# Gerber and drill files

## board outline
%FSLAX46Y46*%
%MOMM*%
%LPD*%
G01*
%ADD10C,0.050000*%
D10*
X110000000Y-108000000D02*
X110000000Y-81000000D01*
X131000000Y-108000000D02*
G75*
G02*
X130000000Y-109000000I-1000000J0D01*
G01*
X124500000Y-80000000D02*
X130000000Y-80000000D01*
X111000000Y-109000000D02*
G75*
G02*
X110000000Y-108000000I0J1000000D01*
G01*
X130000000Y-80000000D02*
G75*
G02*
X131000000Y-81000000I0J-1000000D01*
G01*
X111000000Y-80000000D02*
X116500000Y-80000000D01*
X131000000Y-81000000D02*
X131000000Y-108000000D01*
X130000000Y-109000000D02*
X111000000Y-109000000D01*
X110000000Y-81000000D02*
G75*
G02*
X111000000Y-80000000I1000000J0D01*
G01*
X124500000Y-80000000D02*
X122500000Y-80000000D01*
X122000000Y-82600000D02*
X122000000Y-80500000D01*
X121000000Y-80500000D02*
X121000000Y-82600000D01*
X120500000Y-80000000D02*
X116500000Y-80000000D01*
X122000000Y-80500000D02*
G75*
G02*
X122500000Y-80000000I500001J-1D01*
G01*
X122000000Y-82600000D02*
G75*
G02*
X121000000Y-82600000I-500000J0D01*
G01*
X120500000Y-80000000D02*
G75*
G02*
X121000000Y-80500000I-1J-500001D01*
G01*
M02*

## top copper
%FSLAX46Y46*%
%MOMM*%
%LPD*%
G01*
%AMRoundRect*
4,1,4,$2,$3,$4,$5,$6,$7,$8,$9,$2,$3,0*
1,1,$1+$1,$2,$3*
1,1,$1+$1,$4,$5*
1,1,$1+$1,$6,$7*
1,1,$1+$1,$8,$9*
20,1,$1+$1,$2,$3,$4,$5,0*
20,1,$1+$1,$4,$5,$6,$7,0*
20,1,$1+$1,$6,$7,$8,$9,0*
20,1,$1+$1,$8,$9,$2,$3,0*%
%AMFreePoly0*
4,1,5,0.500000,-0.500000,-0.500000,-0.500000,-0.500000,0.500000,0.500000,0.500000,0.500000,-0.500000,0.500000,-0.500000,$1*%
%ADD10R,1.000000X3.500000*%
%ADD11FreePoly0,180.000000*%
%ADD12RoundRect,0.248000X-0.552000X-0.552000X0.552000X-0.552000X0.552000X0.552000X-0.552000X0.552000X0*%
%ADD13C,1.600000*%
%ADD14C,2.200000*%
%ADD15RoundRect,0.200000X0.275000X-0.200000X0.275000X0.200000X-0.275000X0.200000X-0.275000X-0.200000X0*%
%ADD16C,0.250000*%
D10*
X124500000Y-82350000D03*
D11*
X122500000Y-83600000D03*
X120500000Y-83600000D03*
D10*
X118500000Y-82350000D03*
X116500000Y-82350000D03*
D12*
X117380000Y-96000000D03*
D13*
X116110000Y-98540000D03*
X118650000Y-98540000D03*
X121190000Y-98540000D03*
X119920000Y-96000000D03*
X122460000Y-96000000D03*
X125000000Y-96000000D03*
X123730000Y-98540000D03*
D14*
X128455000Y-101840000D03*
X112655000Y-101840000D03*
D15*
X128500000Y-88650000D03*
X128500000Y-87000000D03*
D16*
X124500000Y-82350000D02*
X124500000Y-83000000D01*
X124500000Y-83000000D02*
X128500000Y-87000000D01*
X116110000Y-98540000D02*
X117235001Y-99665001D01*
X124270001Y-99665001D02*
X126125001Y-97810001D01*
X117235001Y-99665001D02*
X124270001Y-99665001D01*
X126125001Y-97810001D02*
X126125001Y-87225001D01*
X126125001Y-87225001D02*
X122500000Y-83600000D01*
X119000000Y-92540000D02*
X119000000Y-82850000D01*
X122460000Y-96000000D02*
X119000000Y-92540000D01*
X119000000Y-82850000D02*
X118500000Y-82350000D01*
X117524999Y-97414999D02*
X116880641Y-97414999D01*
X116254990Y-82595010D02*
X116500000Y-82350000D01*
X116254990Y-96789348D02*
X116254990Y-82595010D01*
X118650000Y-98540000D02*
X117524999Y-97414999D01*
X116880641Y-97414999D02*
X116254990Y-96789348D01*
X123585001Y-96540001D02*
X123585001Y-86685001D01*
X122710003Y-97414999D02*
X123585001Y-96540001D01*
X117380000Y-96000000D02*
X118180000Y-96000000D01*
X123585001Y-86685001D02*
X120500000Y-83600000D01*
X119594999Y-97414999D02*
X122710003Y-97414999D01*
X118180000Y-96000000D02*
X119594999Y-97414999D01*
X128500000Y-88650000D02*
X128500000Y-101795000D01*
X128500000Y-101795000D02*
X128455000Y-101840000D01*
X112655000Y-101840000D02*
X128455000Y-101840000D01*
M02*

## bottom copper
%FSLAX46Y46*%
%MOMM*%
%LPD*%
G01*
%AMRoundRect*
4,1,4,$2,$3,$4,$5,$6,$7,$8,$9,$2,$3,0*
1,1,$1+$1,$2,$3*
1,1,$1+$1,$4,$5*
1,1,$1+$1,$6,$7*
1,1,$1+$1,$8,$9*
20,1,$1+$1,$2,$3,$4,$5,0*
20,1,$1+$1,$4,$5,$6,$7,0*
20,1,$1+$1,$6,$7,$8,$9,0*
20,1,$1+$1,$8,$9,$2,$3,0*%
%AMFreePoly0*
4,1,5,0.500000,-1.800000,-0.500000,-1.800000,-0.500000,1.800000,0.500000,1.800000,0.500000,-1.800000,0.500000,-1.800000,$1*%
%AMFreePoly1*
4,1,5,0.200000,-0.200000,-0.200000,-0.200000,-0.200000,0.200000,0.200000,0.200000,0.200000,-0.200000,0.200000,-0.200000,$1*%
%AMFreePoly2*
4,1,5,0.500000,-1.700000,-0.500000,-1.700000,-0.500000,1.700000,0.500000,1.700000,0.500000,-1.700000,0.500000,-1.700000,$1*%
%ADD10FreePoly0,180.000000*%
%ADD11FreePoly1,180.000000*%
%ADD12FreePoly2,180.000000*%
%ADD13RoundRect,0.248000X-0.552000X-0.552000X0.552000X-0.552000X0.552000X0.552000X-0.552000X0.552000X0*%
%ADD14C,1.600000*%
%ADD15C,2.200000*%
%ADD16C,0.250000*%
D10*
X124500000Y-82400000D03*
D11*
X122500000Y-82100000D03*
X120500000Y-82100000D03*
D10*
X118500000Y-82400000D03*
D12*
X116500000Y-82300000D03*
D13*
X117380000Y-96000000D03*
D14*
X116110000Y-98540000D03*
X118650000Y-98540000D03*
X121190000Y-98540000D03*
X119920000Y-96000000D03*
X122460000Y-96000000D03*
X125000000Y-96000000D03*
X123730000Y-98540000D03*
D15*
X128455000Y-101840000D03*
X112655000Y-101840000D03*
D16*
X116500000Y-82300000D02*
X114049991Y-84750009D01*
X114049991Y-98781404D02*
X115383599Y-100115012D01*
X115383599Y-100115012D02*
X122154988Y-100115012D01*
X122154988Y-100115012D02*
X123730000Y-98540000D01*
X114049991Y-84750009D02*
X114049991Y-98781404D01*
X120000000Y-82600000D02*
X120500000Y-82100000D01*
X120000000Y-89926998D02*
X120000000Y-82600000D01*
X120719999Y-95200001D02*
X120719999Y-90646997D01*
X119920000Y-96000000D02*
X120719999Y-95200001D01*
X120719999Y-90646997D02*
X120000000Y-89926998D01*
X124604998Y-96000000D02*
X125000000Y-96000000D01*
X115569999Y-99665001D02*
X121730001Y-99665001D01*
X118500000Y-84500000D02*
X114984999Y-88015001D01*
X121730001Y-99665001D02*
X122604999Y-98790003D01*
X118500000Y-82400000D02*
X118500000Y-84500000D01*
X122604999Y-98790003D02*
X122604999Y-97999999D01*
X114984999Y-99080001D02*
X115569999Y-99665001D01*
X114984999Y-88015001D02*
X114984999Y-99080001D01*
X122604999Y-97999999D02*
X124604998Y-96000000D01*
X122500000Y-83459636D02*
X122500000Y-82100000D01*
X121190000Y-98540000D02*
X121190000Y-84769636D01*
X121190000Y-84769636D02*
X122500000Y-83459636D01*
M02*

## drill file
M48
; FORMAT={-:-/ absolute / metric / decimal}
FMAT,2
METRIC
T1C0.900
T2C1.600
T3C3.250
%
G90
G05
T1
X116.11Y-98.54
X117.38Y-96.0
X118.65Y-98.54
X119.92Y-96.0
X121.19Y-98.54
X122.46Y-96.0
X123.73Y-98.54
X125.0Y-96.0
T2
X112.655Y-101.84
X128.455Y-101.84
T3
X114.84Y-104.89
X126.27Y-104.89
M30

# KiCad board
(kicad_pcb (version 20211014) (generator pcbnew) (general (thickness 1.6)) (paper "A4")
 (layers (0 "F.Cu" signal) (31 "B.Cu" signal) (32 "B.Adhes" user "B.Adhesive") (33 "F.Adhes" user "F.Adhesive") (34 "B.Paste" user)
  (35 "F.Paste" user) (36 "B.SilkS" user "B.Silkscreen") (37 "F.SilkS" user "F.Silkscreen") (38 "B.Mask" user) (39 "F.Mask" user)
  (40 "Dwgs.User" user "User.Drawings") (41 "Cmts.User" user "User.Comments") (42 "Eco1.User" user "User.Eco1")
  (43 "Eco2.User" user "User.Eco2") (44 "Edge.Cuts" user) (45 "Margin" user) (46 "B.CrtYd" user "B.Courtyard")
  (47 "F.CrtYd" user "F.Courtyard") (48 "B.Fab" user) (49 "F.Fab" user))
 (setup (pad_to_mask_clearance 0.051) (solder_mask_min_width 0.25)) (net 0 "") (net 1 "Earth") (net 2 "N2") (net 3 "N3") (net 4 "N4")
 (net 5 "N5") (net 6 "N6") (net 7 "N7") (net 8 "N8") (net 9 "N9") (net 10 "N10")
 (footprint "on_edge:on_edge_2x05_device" (layer "F.Cu") (at 120.5 80 180)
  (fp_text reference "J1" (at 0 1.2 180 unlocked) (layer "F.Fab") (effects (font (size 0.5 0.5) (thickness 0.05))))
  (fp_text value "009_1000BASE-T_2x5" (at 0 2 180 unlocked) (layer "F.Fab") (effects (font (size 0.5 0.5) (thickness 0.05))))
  (fp_line (start -4 0) (end -2 0) (layer "Edge.Cuts") (width 0.05))
  (fp_line (start -1.5 -2.6) (end -1.5 -0.5) (layer "Edge.Cuts") (width 0.05))
  (fp_line (start -0.5 -0.5) (end -0.5 -2.6) (layer "Edge.Cuts") (width 0.05))
  (fp_line (start 0 0) (end 4 0) (layer "Edge.Cuts") (width 0.05))
  (fp_arc (start -1.5 -0.5) (mid -1.646447 -0.146447) (end -2 0) (layer "Edge.Cuts") (width 0.05))
  (fp_arc (start -1.5 -2.6) (mid -1 -3.1) (end -0.5 -2.6) (layer "Edge.Cuts") (width 0.05))
  (fp_arc (start 0 0) (mid -0.353553 -0.146447) (end -0.5 -0.5) (layer "Edge.Cuts") (width 0.05))
  (pad "1" smd rect locked (at -4 -2.35) (size 1 3.5) (layers "F.Cu" "F.Mask") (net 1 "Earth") (zone_connect 0))
  (pad "2" smd custom locked (at -2 -3.6 180) (size 1 1) (layers "F.Cu" "F.Mask") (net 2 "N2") (zone_connect 0)
   (options (clearance outline) (anchor rect)) (primitives))
  (pad "3" smd custom locked (at 0 -3.6 180) (size 1 1) (layers "F.Cu" "F.Mask") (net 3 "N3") (zone_connect 0)
   (options (clearance outline) (anchor rect)) (primitives))
  (pad "4" smd rect locked (at 2 -2.35) (size 1 3.5) (layers "F.Cu" "F.Mask") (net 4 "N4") (zone_connect 0))
  (pad "5" smd rect locked (at 4 -2.35) (size 1 3.5) (layers "F.Cu" "F.Mask") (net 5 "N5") (zone_connect 0))
  (pad "6" smd custom locked (at -4 -2.4 180) (size 1 3.6) (layers "B.Cu" "B.Mask") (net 1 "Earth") (zone_connect 0)
   (options (clearance outline) (anchor rect)) (primitives))
  (pad "7" smd custom locked (at -2 -2.1 180) (size 0.4 0.4) (layers "B.Cu" "B.Mask") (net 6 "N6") (zone_connect 0)
   (options (clearance outline) (anchor rect)) (primitives))
  (pad "8" smd custom locked (at 0 -2.1 180) (size 0.4 0.4) (layers "B.Cu" "B.Mask") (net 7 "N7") (zone_connect 0)
   (options (clearance outline) (anchor rect)) (primitives))
  (pad "9" smd custom locked (at 2 -2.4 180) (size 1 3.6) (layers "B.Cu" "B.Mask") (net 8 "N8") (zone_connect 0)
   (options (clearance outline) (anchor rect)) (primitives))
  (pad "10" smd custom locked (at 4 -2.3 180) (size 1 3.4) (layers "B.Cu" "B.Mask") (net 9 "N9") (zone_connect 0)
   (options (clearance outline) (anchor rect)) (primitives)))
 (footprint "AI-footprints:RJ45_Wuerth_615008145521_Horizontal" (layer "F.Cu") (at 125 96 -90)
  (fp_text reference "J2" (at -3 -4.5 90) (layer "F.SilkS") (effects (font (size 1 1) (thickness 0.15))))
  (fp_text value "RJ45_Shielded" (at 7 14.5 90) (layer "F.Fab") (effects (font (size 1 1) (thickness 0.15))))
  (pad "" np_thru_hole circle locked (at 8.89 10.16) (size 3.25 3.25) (drill 3.25) (layers *.Cu *.Mask))
  (pad "" np_thru_hole circle locked (at 8.89 -1.27) (size 3.25 3.25) (drill 3.25) (layers *.Cu *.Mask))
  (pad "1" thru_hole roundrect locked (at 0 7.62) (size 1.6 1.6) (drill 0.9) (layers *.Cu *.Mask) (roundrect_rratio 0.155) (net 3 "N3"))
  (pad "2" thru_hole circle locked (at 2.54 8.89) (size 1.6 1.6) (drill 0.9) (layers *.Cu *.Mask) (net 2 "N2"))
  (pad "3" thru_hole circle locked (at 2.54 6.35) (size 1.6 1.6) (drill 0.9) (layers *.Cu *.Mask) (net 5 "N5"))
  (pad "4" thru_hole circle locked (at 2.54 3.81) (size 1.6 1.6) (drill 0.9) (layers *.Cu *.Mask) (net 6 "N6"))
  (pad "5" thru_hole circle locked (at 0 5.08) (size 1.6 1.6) (drill 0.9) (layers *.Cu *.Mask) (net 7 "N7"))
  (pad "6" thru_hole circle locked (at 0 2.54) (size 1.6 1.6) (drill 0.9) (layers *.Cu *.Mask) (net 4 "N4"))
  (pad "7" thru_hole circle locked (at 0 0) (size 1.6 1.6) (drill 0.9) (layers *.Cu *.Mask) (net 8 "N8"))
  (pad "8" thru_hole circle locked (at 2.54 1.27) (size 1.6 1.6) (drill 0.9) (layers *.Cu *.Mask) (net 9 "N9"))
  (pad "SH" thru_hole circle locked (at 5.84 -3.455) (size 2.2 2.2) (drill 1.6) (layers *.Cu *.Mask) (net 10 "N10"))
  (pad "SH" thru_hole circle locked (at 5.84 12.345) (size 2.2 2.2) (drill 1.6) (layers *.Cu *.Mask) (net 10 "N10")))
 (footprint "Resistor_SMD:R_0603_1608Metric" (layer "F.Cu") (at 128.5 87.825 90)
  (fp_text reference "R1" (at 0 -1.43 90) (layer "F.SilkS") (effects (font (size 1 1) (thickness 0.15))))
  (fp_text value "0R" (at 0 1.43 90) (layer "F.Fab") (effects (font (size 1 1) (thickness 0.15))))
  (pad "1" smd roundrect locked (at -0.825 0 90) (size 0.8 0.95) (layers "F.Cu" "F.Paste" "F.Mask") (roundrect_rratio 0.25) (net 10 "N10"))
  (pad "2" smd roundrect locked (at 0.825 0 90) (size 0.8 0.95) (layers "F.Cu" "F.Paste" "F.Mask") (roundrect_rratio 0.25) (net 1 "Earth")))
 (gr_line (start 110 108) (end 110 81) (layer "Edge.Cuts") (width 0.05))
 (gr_arc (start 131 108) (mid 130.707107 108.707107) (end 130 109) (layer "Edge.Cuts") (width 0.05))
 (gr_line (start 124.5 80) (end 130 80) (layer "Edge.Cuts") (width 0.05))
 (gr_arc (start 111 109) (mid 110.292893 108.707107) (end 110 108) (layer "Edge.Cuts") (width 0.05))
 (gr_arc (start 130 80) (mid 130.707107 80.292893) (end 131 81) (layer "Edge.Cuts") (width 0.05))
 (gr_line (start 111 80) (end 116.5 80) (layer "Edge.Cuts") (width 0.05))
 (gr_line (start 131 81) (end 131 108) (layer "Edge.Cuts") (width 0.05))
 (gr_line (start 130 109) (end 111 109) (layer "Edge.Cuts") (width 0.05))
 (gr_arc (start 110 81) (mid 110.292893 80.292893) (end 111 80) (layer "Edge.Cuts") (width 0.05))
 (segment (start 124.5 82.35) (end 124.5 83) (width 0.25) (layer "F.Cu") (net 1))
 (segment (start 124.5 83) (end 128.5 87) (width 0.25) (layer "F.Cu") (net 1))
 (segment (start 116.11 98.54) (end 117.235001 99.665001) (width 0.25) (layer "F.Cu") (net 2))
 (segment (start 124.270001 99.665001) (end 126.125001 97.810001) (width 0.25) (layer "F.Cu") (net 2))
 (segment (start 117.235001 99.665001) (end 124.270001 99.665001) (width 0.25) (layer "F.Cu") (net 2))
 (segment (start 126.125001 97.810001) (end 126.125001 87.225001) (width 0.25) (layer "F.Cu") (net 2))
 (segment (start 126.125001 87.225001) (end 122.5 83.6) (width 0.25) (layer "F.Cu") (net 2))
 (segment (start 119 92.54) (end 119 82.85) (width 0.25) (layer "F.Cu") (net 4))
 (segment (start 122.46 96) (end 119 92.54) (width 0.25) (layer "F.Cu") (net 4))
 (segment (start 119 82.85) (end 118.5 82.35) (width 0.25) (layer "F.Cu") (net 4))
 (segment (start 116.5 82.3) (end 114.049991 84.750009) (width 0.25) (layer "B.Cu") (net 9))
 (segment (start 114.049991 98.781404) (end 115.383599 100.115012) (width 0.25) (layer "B.Cu") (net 9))
 (segment (start 115.383599 100.115012) (end 122.154988 100.115012) (width 0.25) (layer "B.Cu") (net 9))
 (segment (start 122.154988 100.115012) (end 123.73 98.54) (width 0.25) (layer "B.Cu") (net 9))
 (segment (start 114.049991 84.750009) (end 114.049991 98.781404) (width 0.25) (layer "B.Cu") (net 9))
 (segment (start 120 82.6) (end 120.5 82.1) (width 0.25) (layer "B.Cu") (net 7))
 (segment (start 120 89.926998) (end 120 82.6) (width 0.25) (layer "B.Cu") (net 7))
 (segment (start 120.719999 95.200001) (end 120.719999 90.646997) (width 0.25) (layer "B.Cu") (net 7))
 (segment (start 119.92 96) (end 120.719999 95.200001) (width 0.25) (layer "B.Cu") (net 7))
 (segment (start 120.719999 90.646997) (end 120 89.926998) (width 0.25) (layer "B.Cu") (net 7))
 (segment (start 124.604998 96) (end 125 96) (width 0.25) (layer "B.Cu") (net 8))
 (segment (start 115.569999 99.665001) (end 121.730001 99.665001) (width 0.25) (layer "B.Cu") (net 8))
 (segment (start 118.5 84.5) (end 114.984999 88.015001) (width 0.25) (layer "B.Cu") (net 8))
 (segment (start 121.730001 99.665001) (end 122.604999 98.790003) (width 0.25) (layer "B.Cu") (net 8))
 (segment (start 118.5 82.4) (end 118.5 84.5) (width 0.25) (layer "B.Cu") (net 8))
 (segment (start 122.604999 98.790003) (end 122.604999 97.999999) (width 0.25) (layer "B.Cu") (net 8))
 (segment (start 114.984999 99.080001) (end 115.569999 99.665001) (width 0.25) (layer "B.Cu") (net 8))
 (segment (start 114.984999 88.015001) (end 114.984999 99.080001) (width 0.25) (layer "B.Cu") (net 8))
 (segment (start 122.604999 97.999999) (end 124.604998 96) (width 0.25) (layer "B.Cu") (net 8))
 (segment (start 122.5 83.459636) (end 122.5 82.1) (width 0.25) (layer "B.Cu") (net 6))
 (segment (start 121.19 98.54) (end 121.19 84.769636) (width 0.25) (layer "B.Cu") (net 6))
 (segment (start 121.19 84.769636) (end 122.5 83.459636) (width 0.25) (layer "B.Cu") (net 6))
 (segment (start 117.524999 97.414999) (end 116.880641 97.414999) (width 0.25) (layer "F.Cu") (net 5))
 (segment (start 116.25499 82.59501) (end 116.5 82.35) (width 0.25) (layer "F.Cu") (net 5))
 (segment (start 116.25499 96.789348) (end 116.25499 82.59501) (width 0.25) (layer "F.Cu") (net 5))
 (segment (start 118.65 98.54) (end 117.524999 97.414999) (width 0.25) (layer "F.Cu") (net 5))
 (segment (start 116.880641 97.414999) (end 116.25499 96.789348) (width 0.25) (layer "F.Cu") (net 5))
 (segment (start 123.585001 96.540001) (end 123.585001 86.685001) (width 0.25) (layer "F.Cu") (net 3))
 (segment (start 122.710003 97.414999) (end 123.585001 96.540001) (width 0.25) (layer "F.Cu") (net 3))
 (segment (start 117.38 96) (end 118.18 96) (width 0.25) (layer "F.Cu") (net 3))
 (segment (start 123.585001 86.685001) (end 120.5 83.6) (width 0.25) (layer "F.Cu") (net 3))
 (segment (start 119.594999 97.414999) (end 122.710003 97.414999) (width 0.25) (layer "F.Cu") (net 3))
 (segment (start 118.18 96) (end 119.594999 97.414999) (width 0.25) (layer "F.Cu") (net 3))
 (segment (start 128.5 88.65) (end 128.5 101.795) (width 0.25) (layer "F.Cu") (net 10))
 (segment (start 128.5 101.795) (end 128.455 101.84) (width 0.25) (layer "F.Cu") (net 10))
 (segment (start 112.655 101.84) (end 128.455 101.84) (width 0.25) (layer "F.Cu") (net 10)))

